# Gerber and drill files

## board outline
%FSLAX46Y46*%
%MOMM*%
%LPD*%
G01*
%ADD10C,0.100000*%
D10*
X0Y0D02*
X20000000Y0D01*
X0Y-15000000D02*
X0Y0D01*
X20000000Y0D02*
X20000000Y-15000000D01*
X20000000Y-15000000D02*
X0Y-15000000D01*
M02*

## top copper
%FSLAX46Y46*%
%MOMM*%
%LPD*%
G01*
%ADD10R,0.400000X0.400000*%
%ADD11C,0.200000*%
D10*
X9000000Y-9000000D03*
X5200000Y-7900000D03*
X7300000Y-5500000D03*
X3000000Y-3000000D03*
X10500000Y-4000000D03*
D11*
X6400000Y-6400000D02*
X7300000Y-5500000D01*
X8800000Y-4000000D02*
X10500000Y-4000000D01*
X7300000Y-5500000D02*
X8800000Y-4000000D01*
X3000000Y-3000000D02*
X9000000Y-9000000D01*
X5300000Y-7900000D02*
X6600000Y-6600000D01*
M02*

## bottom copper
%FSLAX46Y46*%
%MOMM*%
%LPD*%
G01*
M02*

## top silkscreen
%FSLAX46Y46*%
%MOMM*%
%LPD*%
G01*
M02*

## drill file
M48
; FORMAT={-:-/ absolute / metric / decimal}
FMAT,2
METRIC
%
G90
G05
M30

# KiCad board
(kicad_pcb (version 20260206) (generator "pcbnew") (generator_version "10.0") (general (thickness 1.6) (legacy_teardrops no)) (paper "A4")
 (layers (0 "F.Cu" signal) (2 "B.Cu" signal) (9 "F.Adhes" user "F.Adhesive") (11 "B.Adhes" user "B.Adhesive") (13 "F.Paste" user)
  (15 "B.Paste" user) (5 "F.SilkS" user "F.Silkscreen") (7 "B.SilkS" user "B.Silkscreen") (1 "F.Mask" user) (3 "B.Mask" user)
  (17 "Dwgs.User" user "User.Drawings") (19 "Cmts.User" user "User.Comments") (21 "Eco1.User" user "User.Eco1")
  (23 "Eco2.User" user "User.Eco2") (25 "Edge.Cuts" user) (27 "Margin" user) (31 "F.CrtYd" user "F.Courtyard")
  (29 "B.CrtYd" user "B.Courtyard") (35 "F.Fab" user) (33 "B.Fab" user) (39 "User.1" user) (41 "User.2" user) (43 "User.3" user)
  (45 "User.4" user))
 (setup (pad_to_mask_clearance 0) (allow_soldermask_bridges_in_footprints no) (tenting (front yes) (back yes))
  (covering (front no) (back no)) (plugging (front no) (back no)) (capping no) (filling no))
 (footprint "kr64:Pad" (layer "F.Cu") (at 9 9)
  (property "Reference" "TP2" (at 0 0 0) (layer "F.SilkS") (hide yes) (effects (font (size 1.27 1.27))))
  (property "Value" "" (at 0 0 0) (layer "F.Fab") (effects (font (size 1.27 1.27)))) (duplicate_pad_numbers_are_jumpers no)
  (pad "1" smd rect (at 0 0) (size 0.4 0.4) (layers "F.Cu" "F.Mask" "F.Paste") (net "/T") (thermal_bridge_angle 45)))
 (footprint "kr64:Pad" (layer "F.Cu") (at 5.2 7.9)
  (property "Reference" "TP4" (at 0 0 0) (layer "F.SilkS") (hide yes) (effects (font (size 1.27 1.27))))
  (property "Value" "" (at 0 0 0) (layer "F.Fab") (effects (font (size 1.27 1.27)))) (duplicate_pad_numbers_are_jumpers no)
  (pad "1" smd rect (at 0 0) (size 0.4 0.4) (layers "F.Cu" "F.Mask" "F.Paste") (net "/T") (thermal_bridge_angle 45)))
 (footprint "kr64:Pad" (layer "F.Cu") (at 7.3 5.5)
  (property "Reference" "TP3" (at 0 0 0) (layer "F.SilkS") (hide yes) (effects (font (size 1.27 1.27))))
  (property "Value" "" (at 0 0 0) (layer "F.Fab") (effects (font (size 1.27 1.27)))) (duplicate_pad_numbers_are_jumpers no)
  (pad "1" smd rect (at 0 0) (size 0.4 0.4) (layers "F.Cu" "F.Mask" "F.Paste") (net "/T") (thermal_bridge_angle 45)))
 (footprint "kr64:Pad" (layer "F.Cu") (at 3 3)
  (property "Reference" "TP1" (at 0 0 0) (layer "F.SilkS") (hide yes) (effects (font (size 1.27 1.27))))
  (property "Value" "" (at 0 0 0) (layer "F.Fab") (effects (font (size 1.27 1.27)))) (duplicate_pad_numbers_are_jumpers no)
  (pad "1" smd rect (at 0 0) (size 0.4 0.4) (layers "F.Cu" "F.Mask" "F.Paste") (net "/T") (thermal_bridge_angle 45)))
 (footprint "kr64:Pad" (layer "F.Cu") (at 10.5 4)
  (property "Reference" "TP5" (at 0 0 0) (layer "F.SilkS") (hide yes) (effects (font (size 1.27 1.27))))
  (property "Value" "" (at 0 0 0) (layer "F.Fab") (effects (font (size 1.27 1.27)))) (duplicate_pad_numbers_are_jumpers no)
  (pad "1" smd rect (at 0 0) (size 0.4 0.4) (layers "F.Cu" "F.Mask" "F.Paste") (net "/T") (thermal_bridge_angle 45)))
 (gr_line (start 0 0) (end 20 0) (stroke (width 0.1) (type default)) (layer "Edge.Cuts"))
 (gr_line (start 0 15) (end 0 0) (stroke (width 0.1) (type default)) (layer "Edge.Cuts"))
 (gr_line (start 20 0) (end 20 15) (stroke (width 0.1) (type default)) (layer "Edge.Cuts"))
 (gr_line (start 20 15) (end 0 15) (stroke (width 0.1) (type default)) (layer "Edge.Cuts"))
 (segment (start 6.4 6.4) (end 7.3 5.5) (width 0.2) (layer "F.Cu") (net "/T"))
 (segment (start 8.8 4) (end 10.5 4) (width 0.2) (layer "F.Cu") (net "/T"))
 (segment (start 7.3 5.5) (end 8.8 4) (width 0.2) (layer "F.Cu") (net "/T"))
 (segment (start 3 3) (end 9 9) (width 0.2) (layer "F.Cu") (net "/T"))
 (segment (start 5.3 7.9) (end 6.6 6.6) (width 0.2) (layer "F.Cu") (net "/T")))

